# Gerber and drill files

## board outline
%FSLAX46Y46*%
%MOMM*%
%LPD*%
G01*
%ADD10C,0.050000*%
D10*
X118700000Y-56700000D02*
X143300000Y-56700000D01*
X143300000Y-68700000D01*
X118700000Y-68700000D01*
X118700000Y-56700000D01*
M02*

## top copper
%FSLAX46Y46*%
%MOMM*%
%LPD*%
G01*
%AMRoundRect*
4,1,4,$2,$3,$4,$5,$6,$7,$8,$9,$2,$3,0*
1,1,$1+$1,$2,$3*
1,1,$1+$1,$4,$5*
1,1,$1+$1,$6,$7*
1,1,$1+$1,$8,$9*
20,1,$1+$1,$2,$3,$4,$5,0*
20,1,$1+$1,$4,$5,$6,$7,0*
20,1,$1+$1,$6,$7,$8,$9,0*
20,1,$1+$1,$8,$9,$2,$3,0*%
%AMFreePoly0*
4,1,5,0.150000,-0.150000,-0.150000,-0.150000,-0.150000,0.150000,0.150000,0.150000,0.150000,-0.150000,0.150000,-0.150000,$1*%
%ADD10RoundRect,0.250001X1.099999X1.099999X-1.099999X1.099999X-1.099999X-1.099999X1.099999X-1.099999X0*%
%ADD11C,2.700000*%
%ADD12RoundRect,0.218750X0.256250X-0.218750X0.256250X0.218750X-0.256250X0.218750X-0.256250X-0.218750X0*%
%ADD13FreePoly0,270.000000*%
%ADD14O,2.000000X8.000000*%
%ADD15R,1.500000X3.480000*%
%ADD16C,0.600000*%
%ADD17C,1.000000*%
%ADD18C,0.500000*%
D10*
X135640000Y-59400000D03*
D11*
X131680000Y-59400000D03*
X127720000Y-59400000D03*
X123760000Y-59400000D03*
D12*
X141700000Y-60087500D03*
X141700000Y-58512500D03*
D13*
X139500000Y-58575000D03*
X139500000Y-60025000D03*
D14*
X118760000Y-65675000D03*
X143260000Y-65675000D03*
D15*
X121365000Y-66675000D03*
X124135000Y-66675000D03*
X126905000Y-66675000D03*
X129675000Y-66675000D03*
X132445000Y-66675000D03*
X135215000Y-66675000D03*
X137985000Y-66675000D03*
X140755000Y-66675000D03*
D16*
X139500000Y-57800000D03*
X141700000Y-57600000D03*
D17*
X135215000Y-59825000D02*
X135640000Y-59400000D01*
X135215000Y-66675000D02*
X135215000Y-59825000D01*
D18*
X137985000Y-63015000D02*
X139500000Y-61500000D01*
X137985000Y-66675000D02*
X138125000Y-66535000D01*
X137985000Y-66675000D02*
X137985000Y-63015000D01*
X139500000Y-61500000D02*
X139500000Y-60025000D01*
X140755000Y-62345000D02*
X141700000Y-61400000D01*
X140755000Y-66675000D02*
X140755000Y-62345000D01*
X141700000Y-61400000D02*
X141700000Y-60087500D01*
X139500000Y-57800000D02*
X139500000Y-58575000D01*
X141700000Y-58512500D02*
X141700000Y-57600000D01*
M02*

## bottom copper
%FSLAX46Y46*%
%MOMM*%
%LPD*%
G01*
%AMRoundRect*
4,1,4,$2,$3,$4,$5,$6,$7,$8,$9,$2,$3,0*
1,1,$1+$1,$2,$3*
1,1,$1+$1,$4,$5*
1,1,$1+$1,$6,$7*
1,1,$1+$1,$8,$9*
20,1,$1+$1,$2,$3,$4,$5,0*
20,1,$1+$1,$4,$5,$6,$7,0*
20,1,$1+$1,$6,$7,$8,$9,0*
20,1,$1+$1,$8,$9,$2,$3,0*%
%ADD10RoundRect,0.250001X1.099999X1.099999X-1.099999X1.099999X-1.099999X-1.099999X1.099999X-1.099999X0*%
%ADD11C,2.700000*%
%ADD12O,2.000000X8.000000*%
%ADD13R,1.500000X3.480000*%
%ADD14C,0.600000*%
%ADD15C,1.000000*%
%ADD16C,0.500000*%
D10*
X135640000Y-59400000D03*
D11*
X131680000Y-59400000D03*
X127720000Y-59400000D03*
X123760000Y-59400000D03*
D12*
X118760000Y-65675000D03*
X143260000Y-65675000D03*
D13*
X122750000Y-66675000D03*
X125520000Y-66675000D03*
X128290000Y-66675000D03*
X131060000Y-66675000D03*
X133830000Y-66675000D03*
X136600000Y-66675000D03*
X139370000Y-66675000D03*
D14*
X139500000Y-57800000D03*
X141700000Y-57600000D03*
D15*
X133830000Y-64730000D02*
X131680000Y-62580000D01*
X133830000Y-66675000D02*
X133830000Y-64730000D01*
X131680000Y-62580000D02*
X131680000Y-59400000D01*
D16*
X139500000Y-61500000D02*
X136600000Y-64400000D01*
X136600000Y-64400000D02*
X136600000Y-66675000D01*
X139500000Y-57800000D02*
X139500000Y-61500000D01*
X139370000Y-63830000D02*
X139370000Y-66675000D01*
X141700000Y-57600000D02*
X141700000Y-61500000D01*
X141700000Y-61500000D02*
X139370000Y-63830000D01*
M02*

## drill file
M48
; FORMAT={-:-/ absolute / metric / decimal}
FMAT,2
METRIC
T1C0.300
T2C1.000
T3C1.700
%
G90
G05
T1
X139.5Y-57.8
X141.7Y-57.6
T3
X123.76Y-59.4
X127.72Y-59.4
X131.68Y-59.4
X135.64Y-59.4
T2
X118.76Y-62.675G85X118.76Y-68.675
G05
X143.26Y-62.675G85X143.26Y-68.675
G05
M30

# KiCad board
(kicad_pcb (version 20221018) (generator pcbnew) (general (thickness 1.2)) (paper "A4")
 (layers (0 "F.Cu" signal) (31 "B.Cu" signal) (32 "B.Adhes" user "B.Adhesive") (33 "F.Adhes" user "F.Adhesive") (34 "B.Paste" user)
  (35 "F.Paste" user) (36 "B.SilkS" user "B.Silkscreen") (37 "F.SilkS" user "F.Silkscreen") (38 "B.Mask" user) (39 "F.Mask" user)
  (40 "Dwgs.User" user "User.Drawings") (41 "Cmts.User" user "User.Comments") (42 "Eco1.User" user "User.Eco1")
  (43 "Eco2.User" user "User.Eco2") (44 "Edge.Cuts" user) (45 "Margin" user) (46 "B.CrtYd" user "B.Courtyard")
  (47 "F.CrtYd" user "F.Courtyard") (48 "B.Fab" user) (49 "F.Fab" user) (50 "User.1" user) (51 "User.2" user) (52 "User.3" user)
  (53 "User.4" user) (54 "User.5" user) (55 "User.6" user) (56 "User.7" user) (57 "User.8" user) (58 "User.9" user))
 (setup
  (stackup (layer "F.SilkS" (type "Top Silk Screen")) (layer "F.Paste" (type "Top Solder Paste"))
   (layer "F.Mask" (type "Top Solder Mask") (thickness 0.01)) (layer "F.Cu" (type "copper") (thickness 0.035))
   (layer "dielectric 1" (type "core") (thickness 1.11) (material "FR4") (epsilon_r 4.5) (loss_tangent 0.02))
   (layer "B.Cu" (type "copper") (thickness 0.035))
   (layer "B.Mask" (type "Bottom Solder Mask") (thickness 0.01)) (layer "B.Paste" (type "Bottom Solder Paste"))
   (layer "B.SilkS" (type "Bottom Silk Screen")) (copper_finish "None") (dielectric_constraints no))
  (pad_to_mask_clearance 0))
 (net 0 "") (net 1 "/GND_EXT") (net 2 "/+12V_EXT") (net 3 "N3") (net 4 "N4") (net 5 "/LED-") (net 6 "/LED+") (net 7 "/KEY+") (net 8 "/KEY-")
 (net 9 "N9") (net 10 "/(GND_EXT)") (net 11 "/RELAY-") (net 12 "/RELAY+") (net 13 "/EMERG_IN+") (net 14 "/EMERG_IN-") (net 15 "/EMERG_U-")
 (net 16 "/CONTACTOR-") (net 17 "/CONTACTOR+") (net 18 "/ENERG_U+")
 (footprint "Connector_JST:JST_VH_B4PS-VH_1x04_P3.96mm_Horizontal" (layer "F.Cu") (at 135.64 59.4 180)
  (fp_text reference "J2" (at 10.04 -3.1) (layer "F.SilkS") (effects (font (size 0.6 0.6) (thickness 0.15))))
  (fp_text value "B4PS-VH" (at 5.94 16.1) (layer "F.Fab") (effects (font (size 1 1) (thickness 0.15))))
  (pad "1" thru_hole roundrect (at 0 0 180) (size 2.7 2.7) (drill 1.7) (layers "*.Cu" "*.Mask") (roundrect_rratio 0.092593)
   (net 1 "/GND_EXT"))
  (pad "2" thru_hole circle (at 3.96 0 180) (size 2.7 2.7) (drill 1.7) (layers "*.Cu" "*.Mask") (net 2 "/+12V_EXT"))
  (pad "3" thru_hole circle (at 7.92 0 180) (size 2.7 2.7) (drill 1.7) (layers "*.Cu" "*.Mask") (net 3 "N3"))
  (pad "4" thru_hole circle (at 11.88 0 180) (size 2.7 2.7) (drill 1.7) (layers "*.Cu" "*.Mask") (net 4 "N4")))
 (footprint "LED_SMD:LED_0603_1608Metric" (layer "F.Cu") (at 141.7 59.3 90)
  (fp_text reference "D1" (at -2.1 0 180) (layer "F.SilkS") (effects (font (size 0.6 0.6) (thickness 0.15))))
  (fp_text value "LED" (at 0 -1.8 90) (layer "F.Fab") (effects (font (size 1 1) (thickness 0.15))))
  (pad "1" smd roundrect (at -0.7875 0 90) (size 0.875 0.95) (layers "F.Cu" "F.Paste" "F.Mask") (roundrect_rratio 0.25) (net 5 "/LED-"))
  (pad "2" smd roundrect (at 0.7875 0 90) (size 0.875 0.95) (layers "F.Cu" "F.Paste" "F.Mask") (roundrect_rratio 0.25) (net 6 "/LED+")))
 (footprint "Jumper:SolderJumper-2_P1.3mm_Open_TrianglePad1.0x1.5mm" (layer "F.Cu") (at 139.5 59.3 -90) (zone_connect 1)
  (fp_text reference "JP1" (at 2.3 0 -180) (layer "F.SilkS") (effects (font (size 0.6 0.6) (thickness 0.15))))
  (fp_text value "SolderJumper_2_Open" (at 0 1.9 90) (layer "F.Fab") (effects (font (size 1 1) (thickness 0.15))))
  (pad "1" smd custom (at -0.725 0 270) (size 0.3 0.3) (layers "F.Cu" "F.Mask") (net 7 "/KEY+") (zone_connect 2) (thermal_bridge_angle 45)
   (options (clearance outline) (anchor rect)) (primitives))
  (pad "2" smd custom (at 0.725 0 270) (size 0.3 0.3) (layers "F.Cu" "F.Mask") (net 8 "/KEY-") (zone_connect 2) (thermal_bridge_angle 45)
   (options (clearance outline) (anchor rect)) (primitives)))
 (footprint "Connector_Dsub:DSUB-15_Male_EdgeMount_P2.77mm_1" (layer "F.Cu") (at 131.06 66.675)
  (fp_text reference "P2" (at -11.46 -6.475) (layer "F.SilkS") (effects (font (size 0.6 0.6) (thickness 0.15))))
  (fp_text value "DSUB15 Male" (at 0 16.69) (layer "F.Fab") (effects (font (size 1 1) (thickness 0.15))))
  (pad "0" thru_hole oval (at -12.3 -1) (size 2 8) (drill oval 1 7) (layers "*.Cu" "*.Mask") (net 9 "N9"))
  (pad "0" thru_hole oval (at 12.2 -1) (size 2 8) (drill oval 1 7) (layers "*.Cu" "*.Mask") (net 9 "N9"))
  (pad "1" smd rect (at -9.695 0) (size 1.5 3.48) (layers "F.Cu" "F.Paste" "F.Mask") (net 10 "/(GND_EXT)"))
  (pad "2" smd rect (at -6.925 0) (size 1.5 3.48) (layers "F.Cu" "F.Paste" "F.Mask") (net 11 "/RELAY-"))
  (pad "3" smd rect (at -4.155 0) (size 1.5 3.48) (layers "F.Cu" "F.Paste" "F.Mask") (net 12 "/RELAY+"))
  (pad "4" smd rect (at -1.385 0) (size 1.5 3.48) (layers "F.Cu" "F.Paste" "F.Mask") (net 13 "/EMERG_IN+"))
  (pad "5" smd rect (at 1.385 0) (size 1.5 3.48) (layers "F.Cu" "F.Paste" "F.Mask") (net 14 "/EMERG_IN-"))
  (pad "6" smd rect (at 4.155 0) (size 1.5 3.48) (layers "F.Cu" "F.Paste" "F.Mask") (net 1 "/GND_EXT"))
  (pad "7" smd rect (at 6.925 0) (size 1.5 3.48) (layers "F.Cu" "F.Paste" "F.Mask") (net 8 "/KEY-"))
  (pad "8" smd rect (at 9.695 0) (size 1.5 3.48) (layers "F.Cu" "F.Paste" "F.Mask") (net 5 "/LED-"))
  (pad "9" smd rect (at -8.31 0) (size 1.5 3.48) (layers "B.Cu" "B.Paste" "B.Mask") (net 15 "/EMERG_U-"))
  (pad "10" smd rect (at -5.54 0) (size 1.5 3.48) (layers "B.Cu" "B.Paste" "B.Mask") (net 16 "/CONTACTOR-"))
  (pad "11" smd rect (at -2.77 0) (size 1.5 3.48) (layers "B.Cu" "B.Paste" "B.Mask") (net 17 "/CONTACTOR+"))
  (pad "12" smd rect (at 0 0) (size 1.5 3.48) (layers "B.Cu" "B.Paste" "B.Mask") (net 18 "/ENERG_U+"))
  (pad "13" smd rect (at 2.77 0) (size 1.5 3.48) (layers "B.Cu" "B.Paste" "B.Mask") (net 2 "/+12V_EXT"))
  (pad "14" smd rect (at 5.54 0) (size 1.5 3.48) (layers "B.Cu" "B.Paste" "B.Mask") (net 7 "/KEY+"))
  (pad "15" smd rect (at 8.31 0) (size 1.5 3.48) (layers "B.Cu" "B.Paste" "B.Mask") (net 6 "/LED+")))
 (gr_rect (start 118.7 56.7) (end 143.3 68.7) (stroke (width 0.05) (type default)) (fill none) (layer "Edge.Cuts"))
 (segment (start 135.215 59.825) (end 135.64 59.4) (width 1) (layer "F.Cu") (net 1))
 (segment (start 135.215 66.675) (end 135.215 59.825) (width 1) (layer "F.Cu") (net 1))
 (segment (start 137.985 63.015) (end 139.5 61.5) (width 0.5) (layer "F.Cu") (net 8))
 (segment (start 137.985 66.675) (end 138.125 66.535) (width 0.5) (layer "F.Cu") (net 8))
 (segment (start 137.985 66.675) (end 137.985 63.015) (width 0.5) (layer "F.Cu") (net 8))
 (segment (start 139.5 61.5) (end 139.5 60.025) (width 0.5) (layer "F.Cu") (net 8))
 (segment (start 140.755 62.345) (end 141.7 61.4) (width 0.5) (layer "F.Cu") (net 5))
 (segment (start 140.755 66.675) (end 140.755 62.345) (width 0.5) (layer "F.Cu") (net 5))
 (segment (start 141.7 61.4) (end 141.7 60.0875) (width 0.5) (layer "F.Cu") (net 5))
 (segment (start 133.83 64.73) (end 131.68 62.58) (width 1) (layer "B.Cu") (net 2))
 (segment (start 133.83 66.675) (end 133.83 64.73) (width 1) (layer "B.Cu") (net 2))
 (segment (start 131.68 62.58) (end 131.68 59.4) (width 1) (layer "B.Cu") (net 2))
 (segment (start 139.5 57.8) (end 139.5 58.575) (width 0.5) (layer "F.Cu") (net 7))
 (via (at 139.5 57.8) (size 0.6) (drill 0.3) (layers "F.Cu" "B.Cu") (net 7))
 (segment (start 139.5 61.5) (end 136.6 64.4) (width 0.5) (layer "B.Cu") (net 7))
 (segment (start 136.6 64.4) (end 136.6 66.675) (width 0.5) (layer "B.Cu") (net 7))
 (segment (start 139.5 57.8) (end 139.5 61.5) (width 0.5) (layer "B.Cu") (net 7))
 (segment (start 141.7 58.5125) (end 141.7 57.6) (width 0.5) (layer "F.Cu") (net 6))
 (via (at 141.7 57.6) (size 0.6) (drill 0.3) (layers "F.Cu" "B.Cu") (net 6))
 (segment (start 139.37 63.83) (end 139.37 66.675) (width 0.5) (layer "B.Cu") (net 6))
 (segment (start 141.7 57.6) (end 141.7 61.5) (width 0.5) (layer "B.Cu") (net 6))
 (segment (start 141.7 61.5) (end 139.37 63.83) (width 0.5) (layer "B.Cu") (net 6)))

